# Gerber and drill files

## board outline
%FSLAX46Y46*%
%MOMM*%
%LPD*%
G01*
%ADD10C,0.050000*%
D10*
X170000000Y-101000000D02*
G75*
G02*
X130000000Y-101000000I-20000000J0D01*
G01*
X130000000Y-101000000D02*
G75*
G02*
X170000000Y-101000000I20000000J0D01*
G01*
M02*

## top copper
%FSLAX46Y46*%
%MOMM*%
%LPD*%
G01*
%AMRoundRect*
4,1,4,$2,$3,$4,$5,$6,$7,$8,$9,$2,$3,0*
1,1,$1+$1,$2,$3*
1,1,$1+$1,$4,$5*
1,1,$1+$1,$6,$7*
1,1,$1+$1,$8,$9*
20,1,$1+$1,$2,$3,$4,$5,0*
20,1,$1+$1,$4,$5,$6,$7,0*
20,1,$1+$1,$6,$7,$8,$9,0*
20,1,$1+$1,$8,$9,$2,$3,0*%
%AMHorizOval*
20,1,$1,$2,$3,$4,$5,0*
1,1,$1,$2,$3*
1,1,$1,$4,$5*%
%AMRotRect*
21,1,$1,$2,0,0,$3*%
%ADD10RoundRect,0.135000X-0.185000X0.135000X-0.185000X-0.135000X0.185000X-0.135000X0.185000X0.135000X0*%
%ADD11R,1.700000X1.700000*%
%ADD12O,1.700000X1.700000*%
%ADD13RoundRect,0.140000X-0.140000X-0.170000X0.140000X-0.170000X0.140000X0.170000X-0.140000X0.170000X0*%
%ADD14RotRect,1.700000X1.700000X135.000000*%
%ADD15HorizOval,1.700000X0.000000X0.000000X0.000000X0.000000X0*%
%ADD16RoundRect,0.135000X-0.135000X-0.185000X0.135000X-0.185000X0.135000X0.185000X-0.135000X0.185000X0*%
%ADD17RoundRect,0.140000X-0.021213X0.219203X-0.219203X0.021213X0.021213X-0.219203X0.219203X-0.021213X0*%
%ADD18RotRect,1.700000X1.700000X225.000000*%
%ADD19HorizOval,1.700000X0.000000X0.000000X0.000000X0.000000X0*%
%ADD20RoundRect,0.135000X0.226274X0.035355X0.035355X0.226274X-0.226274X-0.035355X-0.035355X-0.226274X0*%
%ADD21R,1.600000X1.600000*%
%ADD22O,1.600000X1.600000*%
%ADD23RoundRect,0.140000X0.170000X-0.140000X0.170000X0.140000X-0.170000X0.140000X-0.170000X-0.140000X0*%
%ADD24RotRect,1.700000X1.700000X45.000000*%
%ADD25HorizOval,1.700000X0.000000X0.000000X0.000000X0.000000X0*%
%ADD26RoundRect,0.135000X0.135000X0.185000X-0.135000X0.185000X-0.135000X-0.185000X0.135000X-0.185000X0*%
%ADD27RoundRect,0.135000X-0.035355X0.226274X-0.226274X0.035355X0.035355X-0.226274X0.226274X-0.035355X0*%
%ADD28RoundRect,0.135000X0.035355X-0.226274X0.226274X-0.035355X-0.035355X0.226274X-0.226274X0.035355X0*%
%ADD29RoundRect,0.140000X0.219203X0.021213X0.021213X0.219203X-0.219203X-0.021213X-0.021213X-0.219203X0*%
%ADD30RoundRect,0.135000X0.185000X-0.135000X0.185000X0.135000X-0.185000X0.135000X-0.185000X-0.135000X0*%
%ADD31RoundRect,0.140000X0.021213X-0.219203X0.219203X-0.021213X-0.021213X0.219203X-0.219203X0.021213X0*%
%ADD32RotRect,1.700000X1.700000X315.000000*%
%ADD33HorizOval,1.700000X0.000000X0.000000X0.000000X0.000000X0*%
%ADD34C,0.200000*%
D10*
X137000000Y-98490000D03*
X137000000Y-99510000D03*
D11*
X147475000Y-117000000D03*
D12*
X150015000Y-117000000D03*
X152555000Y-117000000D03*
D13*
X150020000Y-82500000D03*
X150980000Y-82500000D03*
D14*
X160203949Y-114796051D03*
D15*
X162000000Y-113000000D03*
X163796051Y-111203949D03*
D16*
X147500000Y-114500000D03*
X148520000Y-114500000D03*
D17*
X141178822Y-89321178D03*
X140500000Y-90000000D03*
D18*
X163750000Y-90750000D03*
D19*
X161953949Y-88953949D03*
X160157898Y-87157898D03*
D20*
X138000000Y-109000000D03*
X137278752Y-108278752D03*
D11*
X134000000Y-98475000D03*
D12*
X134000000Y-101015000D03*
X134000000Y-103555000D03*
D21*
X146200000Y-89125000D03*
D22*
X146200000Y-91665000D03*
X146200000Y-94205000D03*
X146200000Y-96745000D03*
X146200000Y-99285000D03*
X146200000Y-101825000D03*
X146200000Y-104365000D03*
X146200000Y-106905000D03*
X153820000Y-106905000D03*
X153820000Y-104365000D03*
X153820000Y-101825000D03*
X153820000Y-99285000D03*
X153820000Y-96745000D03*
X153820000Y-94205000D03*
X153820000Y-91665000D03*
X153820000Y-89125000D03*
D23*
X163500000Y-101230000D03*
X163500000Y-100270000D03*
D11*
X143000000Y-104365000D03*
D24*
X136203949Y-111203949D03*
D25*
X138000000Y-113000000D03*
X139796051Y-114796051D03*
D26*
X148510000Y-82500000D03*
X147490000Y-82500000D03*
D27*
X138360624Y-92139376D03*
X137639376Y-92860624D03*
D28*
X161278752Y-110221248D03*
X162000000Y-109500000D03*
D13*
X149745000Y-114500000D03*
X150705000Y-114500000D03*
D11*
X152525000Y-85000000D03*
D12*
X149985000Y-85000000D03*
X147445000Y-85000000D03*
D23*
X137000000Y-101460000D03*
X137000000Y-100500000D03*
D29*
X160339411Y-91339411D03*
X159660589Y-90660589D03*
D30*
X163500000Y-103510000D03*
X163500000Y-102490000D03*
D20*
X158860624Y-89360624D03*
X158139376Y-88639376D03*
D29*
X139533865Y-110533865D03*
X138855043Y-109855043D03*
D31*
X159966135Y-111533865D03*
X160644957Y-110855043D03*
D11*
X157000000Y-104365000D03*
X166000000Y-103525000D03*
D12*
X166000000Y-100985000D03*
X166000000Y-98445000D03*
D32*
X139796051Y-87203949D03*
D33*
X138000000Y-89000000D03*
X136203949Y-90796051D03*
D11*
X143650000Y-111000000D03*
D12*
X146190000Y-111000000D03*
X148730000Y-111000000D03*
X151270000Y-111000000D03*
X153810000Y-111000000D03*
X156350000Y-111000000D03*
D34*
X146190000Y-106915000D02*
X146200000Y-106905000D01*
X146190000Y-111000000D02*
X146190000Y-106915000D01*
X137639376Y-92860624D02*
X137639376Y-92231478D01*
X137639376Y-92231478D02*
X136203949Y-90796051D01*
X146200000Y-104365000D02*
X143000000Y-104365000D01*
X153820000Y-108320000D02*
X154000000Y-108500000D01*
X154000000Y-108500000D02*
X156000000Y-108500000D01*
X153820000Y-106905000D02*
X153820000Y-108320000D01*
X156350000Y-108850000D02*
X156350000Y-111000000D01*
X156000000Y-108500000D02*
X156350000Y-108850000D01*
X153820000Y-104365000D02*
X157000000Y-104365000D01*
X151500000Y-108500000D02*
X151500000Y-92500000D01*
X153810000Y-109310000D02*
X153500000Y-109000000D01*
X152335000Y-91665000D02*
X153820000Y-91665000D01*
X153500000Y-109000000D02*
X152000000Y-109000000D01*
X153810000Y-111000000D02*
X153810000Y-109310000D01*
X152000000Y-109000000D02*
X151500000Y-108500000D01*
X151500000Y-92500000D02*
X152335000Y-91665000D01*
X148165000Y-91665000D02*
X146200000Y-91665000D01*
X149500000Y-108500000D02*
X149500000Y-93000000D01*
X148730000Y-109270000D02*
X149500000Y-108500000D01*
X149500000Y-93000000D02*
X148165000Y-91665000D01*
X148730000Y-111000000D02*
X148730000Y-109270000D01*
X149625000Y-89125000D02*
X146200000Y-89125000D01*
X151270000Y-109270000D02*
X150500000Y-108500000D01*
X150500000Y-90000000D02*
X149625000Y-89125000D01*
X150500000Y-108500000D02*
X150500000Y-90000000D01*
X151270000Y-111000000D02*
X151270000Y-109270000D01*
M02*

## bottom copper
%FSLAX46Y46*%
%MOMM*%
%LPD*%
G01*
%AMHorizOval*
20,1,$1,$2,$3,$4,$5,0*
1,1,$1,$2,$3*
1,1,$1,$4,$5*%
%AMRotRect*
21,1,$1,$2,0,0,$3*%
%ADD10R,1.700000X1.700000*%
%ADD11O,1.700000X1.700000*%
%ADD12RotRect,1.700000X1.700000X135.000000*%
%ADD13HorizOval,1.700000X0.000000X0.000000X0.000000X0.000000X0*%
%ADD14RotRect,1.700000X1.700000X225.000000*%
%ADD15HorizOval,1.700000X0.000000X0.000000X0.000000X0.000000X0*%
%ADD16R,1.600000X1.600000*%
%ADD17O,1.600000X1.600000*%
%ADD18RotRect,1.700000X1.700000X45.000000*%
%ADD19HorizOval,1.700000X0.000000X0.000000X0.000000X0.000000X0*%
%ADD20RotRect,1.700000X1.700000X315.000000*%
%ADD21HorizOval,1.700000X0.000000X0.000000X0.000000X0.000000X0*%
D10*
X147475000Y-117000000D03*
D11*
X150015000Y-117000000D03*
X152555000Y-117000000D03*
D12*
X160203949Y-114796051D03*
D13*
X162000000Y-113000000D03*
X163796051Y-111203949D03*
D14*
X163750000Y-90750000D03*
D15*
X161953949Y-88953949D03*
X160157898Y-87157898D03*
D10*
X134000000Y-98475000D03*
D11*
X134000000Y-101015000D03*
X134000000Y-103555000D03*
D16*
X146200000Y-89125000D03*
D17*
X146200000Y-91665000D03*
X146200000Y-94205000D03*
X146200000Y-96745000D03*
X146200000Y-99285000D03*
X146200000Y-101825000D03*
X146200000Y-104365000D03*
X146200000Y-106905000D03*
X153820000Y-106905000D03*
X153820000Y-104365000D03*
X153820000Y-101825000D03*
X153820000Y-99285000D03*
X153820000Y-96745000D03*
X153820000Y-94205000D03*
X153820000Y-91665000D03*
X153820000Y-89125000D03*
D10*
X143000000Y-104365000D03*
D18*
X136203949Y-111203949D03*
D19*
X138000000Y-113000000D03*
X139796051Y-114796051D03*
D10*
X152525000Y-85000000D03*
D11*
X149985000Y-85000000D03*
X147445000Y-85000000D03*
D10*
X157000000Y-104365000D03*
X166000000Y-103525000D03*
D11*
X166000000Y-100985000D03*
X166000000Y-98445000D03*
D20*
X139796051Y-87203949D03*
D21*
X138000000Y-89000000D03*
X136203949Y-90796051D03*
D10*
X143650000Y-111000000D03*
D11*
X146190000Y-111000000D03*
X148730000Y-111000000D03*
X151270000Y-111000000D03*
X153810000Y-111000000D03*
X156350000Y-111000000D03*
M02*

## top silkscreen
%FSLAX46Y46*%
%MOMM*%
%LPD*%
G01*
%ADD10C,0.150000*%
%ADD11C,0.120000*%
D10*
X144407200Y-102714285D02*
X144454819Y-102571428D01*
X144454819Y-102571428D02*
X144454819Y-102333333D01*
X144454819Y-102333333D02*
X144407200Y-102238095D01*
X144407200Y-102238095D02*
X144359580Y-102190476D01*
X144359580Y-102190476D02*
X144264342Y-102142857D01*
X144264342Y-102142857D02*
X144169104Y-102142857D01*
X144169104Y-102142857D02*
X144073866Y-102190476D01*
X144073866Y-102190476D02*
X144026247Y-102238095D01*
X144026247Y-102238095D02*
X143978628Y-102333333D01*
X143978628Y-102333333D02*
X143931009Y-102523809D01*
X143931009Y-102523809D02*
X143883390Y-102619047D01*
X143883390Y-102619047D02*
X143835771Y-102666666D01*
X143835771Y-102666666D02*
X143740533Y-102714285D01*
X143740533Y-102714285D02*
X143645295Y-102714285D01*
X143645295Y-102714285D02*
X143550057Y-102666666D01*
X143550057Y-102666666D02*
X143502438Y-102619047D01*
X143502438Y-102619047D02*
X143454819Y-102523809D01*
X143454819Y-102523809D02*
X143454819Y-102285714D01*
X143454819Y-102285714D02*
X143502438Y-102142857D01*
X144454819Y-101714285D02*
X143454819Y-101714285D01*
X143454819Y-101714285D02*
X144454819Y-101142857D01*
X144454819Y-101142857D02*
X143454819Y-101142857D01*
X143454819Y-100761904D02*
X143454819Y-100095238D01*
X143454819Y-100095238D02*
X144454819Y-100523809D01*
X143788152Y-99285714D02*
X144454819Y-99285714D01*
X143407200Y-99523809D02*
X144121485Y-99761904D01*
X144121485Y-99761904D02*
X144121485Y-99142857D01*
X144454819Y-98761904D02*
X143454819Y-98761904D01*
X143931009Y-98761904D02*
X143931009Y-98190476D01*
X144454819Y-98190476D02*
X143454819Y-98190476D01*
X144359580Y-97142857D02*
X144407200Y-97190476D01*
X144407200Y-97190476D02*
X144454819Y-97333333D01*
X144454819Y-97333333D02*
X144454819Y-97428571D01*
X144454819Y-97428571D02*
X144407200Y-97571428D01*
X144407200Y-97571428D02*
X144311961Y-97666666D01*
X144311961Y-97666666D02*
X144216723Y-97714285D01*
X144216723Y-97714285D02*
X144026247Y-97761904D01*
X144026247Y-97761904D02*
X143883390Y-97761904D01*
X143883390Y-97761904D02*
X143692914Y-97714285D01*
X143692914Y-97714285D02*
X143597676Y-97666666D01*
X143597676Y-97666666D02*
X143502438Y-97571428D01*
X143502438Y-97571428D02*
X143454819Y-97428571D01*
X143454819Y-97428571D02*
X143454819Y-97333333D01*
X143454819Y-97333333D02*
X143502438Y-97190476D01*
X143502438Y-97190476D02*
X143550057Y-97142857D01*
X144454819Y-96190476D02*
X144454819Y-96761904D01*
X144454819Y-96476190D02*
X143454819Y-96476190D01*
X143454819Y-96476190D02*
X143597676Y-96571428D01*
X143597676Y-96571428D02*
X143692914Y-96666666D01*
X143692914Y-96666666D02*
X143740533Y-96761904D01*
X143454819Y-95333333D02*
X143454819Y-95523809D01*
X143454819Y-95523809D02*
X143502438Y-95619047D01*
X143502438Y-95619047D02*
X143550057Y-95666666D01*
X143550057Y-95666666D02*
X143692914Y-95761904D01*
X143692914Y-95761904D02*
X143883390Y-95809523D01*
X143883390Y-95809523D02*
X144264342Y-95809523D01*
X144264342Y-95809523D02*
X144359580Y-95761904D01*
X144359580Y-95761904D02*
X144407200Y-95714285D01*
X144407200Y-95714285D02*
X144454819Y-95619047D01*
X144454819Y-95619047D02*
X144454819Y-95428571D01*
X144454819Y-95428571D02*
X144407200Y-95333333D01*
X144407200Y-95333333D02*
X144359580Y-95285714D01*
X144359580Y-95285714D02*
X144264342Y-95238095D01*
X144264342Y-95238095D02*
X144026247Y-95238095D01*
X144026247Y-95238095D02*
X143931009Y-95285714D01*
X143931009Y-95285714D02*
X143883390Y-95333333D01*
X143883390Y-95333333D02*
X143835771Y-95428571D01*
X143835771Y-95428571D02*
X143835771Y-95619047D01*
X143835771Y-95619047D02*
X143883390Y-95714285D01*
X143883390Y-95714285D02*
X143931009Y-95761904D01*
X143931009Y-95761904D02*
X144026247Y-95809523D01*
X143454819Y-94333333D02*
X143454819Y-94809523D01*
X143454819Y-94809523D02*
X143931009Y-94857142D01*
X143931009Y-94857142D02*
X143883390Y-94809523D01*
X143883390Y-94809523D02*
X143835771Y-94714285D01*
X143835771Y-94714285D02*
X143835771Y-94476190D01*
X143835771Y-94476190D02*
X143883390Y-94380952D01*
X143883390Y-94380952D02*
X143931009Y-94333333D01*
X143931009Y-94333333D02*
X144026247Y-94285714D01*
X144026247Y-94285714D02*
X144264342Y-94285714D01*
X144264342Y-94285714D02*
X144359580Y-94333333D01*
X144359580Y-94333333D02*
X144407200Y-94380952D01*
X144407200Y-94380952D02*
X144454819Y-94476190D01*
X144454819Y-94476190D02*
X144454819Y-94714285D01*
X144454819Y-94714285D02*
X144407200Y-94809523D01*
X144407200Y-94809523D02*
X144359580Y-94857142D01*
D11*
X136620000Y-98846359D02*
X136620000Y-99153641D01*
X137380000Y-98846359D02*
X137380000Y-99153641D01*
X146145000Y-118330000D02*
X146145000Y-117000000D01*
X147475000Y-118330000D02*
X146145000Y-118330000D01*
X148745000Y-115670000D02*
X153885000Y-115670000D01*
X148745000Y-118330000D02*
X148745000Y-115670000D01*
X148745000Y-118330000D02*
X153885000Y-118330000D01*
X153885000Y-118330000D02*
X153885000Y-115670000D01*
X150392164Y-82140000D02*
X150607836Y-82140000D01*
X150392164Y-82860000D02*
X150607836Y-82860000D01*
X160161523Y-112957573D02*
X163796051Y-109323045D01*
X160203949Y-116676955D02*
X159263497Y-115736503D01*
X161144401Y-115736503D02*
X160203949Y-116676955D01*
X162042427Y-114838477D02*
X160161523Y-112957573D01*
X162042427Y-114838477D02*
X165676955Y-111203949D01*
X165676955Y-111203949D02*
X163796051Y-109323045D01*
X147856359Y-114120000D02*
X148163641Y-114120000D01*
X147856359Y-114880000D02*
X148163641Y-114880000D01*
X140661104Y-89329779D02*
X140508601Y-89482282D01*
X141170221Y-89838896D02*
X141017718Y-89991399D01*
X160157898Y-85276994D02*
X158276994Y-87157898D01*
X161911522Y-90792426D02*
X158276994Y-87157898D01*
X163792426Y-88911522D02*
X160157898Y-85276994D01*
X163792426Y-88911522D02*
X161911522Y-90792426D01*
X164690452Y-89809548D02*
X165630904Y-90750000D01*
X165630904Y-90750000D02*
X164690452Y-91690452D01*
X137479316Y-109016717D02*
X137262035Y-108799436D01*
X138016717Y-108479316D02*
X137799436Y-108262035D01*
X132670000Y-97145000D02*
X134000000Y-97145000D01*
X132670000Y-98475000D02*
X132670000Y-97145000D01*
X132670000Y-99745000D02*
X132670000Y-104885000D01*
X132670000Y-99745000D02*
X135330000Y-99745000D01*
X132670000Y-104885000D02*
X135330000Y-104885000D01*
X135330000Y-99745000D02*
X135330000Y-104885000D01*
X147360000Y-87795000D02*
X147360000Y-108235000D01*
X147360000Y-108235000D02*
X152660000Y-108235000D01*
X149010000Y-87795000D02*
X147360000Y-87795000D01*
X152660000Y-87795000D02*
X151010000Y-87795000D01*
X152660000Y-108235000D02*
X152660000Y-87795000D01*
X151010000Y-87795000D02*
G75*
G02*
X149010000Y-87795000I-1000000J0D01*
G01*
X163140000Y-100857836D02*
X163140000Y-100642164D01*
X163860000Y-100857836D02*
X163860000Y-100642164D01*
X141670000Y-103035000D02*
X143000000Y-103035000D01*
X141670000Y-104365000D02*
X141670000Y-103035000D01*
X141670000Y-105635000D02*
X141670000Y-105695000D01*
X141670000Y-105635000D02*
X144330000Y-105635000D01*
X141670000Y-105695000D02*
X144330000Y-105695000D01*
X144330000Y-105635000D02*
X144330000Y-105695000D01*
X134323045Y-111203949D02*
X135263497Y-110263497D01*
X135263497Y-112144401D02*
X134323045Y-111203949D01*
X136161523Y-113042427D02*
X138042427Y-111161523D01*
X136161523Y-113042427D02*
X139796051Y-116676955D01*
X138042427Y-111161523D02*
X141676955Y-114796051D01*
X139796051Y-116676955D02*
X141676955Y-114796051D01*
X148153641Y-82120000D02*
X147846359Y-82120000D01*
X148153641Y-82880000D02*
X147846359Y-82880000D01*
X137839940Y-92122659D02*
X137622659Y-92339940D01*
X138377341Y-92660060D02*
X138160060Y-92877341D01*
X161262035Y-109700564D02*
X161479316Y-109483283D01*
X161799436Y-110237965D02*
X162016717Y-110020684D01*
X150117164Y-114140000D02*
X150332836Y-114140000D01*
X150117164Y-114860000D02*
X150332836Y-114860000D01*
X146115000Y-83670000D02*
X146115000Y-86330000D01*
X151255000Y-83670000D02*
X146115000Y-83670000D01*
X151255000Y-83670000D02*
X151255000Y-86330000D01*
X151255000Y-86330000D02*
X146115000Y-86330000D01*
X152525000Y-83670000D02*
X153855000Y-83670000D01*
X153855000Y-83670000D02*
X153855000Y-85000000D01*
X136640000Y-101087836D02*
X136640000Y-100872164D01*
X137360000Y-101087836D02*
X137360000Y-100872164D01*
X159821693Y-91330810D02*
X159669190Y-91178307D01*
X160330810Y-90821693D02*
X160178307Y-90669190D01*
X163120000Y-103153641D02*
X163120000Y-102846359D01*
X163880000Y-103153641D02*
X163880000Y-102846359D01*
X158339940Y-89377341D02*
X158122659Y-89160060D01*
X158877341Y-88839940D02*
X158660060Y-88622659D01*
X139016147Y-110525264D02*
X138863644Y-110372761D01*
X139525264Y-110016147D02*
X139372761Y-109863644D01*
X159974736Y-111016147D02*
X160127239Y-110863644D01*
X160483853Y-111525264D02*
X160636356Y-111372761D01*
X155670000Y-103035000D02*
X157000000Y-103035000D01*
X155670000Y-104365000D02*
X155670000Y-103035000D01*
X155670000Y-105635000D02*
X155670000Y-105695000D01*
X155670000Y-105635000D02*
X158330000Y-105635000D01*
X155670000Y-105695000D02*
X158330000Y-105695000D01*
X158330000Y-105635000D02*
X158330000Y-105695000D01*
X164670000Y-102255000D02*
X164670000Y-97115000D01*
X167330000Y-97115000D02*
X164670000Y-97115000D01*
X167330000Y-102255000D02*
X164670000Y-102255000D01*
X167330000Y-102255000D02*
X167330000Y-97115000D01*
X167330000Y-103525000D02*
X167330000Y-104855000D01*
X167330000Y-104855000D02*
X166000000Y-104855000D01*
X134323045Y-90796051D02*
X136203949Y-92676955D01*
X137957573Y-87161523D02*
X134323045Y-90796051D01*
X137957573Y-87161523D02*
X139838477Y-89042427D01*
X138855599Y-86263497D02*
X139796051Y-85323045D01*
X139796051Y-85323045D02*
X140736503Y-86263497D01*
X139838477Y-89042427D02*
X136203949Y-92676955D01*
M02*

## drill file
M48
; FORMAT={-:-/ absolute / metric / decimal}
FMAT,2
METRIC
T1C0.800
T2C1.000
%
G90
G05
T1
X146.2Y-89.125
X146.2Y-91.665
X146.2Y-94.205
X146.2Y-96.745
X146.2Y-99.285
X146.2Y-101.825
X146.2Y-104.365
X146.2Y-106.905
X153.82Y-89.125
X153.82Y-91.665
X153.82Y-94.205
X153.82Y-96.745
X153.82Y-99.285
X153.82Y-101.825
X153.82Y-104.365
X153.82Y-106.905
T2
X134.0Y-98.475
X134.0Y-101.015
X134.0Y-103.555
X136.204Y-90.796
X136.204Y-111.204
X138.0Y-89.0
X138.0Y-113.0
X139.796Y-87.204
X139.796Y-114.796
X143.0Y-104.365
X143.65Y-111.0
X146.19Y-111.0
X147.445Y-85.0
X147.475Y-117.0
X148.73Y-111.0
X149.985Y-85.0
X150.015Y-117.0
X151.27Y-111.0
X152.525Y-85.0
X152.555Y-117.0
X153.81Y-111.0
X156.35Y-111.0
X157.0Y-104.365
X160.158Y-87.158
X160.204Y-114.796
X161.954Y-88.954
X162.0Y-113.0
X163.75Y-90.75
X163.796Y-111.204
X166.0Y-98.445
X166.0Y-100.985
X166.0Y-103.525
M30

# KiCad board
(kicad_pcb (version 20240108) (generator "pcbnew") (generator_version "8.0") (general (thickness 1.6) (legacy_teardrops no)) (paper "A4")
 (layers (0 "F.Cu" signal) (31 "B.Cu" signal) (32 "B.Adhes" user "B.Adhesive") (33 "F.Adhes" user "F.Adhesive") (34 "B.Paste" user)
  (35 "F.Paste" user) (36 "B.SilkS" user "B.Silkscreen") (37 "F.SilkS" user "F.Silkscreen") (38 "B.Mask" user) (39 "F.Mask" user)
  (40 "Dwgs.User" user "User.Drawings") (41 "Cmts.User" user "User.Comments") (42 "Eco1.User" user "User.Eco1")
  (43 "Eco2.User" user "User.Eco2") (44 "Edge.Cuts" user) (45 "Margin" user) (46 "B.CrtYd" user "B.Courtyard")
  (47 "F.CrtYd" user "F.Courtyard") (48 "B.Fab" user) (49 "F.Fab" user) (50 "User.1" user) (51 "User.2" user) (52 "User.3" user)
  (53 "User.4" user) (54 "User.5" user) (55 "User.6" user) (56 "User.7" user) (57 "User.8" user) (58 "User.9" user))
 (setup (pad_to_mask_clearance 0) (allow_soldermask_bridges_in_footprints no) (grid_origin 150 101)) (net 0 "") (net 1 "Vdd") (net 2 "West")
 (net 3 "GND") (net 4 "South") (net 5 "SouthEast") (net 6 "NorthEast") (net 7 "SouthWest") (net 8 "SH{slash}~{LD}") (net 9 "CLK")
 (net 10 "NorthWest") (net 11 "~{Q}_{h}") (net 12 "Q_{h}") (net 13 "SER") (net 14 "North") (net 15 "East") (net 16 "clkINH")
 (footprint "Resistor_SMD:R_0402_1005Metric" (layer "F.Cu") (at 137 99 -90)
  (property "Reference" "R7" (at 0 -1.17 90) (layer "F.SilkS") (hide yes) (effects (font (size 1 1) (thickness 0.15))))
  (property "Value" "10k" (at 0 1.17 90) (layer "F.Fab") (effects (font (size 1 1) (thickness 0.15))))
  (fp_line (start -0.153641 0.38) (end 0.153641 0.38) (stroke (width 0.12) (type solid)) (layer "F.SilkS"))
  (fp_line (start -0.153641 -0.38) (end 0.153641 -0.38) (stroke (width 0.12) (type solid)) (layer "F.SilkS"))
  (pad "1" smd roundrect (at -0.51 0 270) (size 0.54 0.64) (layers "F.Cu" "F.Paste" "F.Mask") (roundrect_rratio 0.25) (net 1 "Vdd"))
  (pad "2" smd roundrect (at 0.51 0 270) (size 0.54 0.64) (layers "F.Cu" "F.Paste" "F.Mask") (roundrect_rratio 0.25) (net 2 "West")))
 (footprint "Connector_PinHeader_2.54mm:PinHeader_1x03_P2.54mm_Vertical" (layer "F.Cu") (at 147.475 117 90)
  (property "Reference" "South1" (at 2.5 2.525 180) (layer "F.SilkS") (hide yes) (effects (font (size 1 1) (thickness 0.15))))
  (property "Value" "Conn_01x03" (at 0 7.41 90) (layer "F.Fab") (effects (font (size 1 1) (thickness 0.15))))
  (fp_line (start -1.33 -1.33) (end 0 -1.33) (stroke (width 0.12) (type solid)) (layer "F.SilkS"))
  (fp_line (start -1.33 0) (end -1.33 -1.33) (stroke (width 0.12) (type solid)) (layer "F.SilkS"))
  (fp_line (start 1.33 1.27) (end 1.33 6.41) (stroke (width 0.12) (type solid)) (layer "F.SilkS"))
  (fp_line (start -1.33 1.27) (end 1.33 1.27) (stroke (width 0.12) (type solid)) (layer "F.SilkS"))
  (fp_line (start -1.33 1.27) (end -1.33 6.41) (stroke (width 0.12) (type solid)) (layer "F.SilkS"))
  (fp_line (start -1.33 6.41) (end 1.33 6.41) (stroke (width 0.12) (type solid)) (layer "F.SilkS"))
  (pad "1" thru_hole rect (at 0 0 90) (size 1.7 1.7) (drill 1) (layers "*.Cu" "*.Mask") (remove_unused_layers no) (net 1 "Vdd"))
  (pad "2" thru_hole oval (at 0 2.54 90) (size 1.7 1.7) (drill 1) (layers "*.Cu" "*.Mask") (remove_unused_layers no) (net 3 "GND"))
  (pad "3" thru_hole oval (at 0 5.08 90) (size 1.7 1.7) (drill 1) (layers "*.Cu" "*.Mask") (remove_unused_layers no) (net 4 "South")))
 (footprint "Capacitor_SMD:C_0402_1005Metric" (layer "F.Cu") (at 150.5 82.5)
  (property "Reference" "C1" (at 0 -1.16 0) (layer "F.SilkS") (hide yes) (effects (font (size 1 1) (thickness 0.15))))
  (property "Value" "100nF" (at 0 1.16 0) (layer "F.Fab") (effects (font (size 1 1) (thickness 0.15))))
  (fp_line (start -0.107836 -0.36) (end 0.107836 -0.36) (stroke (width 0.12) (type solid)) (layer "F.SilkS"))
  (fp_line (start -0.107836 0.36) (end 0.107836 0.36) (stroke (width 0.12) (type solid)) (layer "F.SilkS"))
  (pad "1" smd roundrect (at -0.48 0) (size 0.56 0.62) (layers "F.Cu" "F.Paste" "F.Mask") (roundrect_rratio 0.25) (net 3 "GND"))
  (pad "2" smd roundrect (at 0.48 0) (size 0.56 0.62) (layers "F.Cu" "F.Paste" "F.Mask") (roundrect_rratio 0.25) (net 1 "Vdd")))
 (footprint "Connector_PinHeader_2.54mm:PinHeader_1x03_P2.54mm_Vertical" (layer "F.Cu") (at 160.203949 114.796051 135)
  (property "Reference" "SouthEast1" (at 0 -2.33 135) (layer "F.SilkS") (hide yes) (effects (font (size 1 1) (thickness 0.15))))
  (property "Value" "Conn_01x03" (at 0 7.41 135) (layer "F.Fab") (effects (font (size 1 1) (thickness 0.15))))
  (fp_line (start 1.33 1.270001) (end 1.33 6.409999) (stroke (width 0.12) (type solid)) (layer "F.SilkS"))
  (fp_line (start -1.33 -1.33) (end 0 -1.33) (stroke (width 0.12) (type solid)) (layer "F.SilkS"))
  (fp_line (start -1.33 0) (end -1.33 -1.33) (stroke (width 0.12) (type solid)) (layer "F.SilkS"))
  (fp_line (start -1.33 1.270001) (end 1.33 1.270001) (stroke (width 0.12) (type solid)) (layer "F.SilkS"))
  (fp_line (start -1.33 1.270001) (end -1.33 6.409999) (stroke (width 0.12) (type solid)) (layer "F.SilkS"))
  (fp_line (start -1.33 6.409999) (end 1.33 6.409999) (stroke (width 0.12) (type solid)) (layer "F.SilkS"))
  (pad "1" thru_hole rect (at 0 0 135) (size 1.7 1.7) (drill 1) (layers "*.Cu" "*.Mask") (remove_unused_layers no) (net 1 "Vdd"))
  (pad "2" thru_hole oval (at 0 2.54 135) (size 1.7 1.7) (drill 1) (layers "*.Cu" "*.Mask") (remove_unused_layers no) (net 3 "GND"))
  (pad "3" thru_hole oval (at 0 5.079999 135) (size 1.7 1.7) (drill 1) (layers "*.Cu" "*.Mask") (remove_unused_layers no)
   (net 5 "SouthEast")))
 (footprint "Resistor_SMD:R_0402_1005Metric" (layer "F.Cu") (at 148.01 114.5)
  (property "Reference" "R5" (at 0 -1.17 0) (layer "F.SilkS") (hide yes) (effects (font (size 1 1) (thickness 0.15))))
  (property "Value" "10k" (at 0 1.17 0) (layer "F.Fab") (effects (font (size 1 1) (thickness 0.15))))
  (fp_line (start -0.153641 -0.38) (end 0.153641 -0.38) (stroke (width 0.12) (type solid)) (layer "F.SilkS"))
  (fp_line (start -0.153641 0.38) (end 0.153641 0.38) (stroke (width 0.12) (type solid)) (layer "F.SilkS"))
  (pad "1" smd roundrect (at -0.51 0) (size 0.54 0.64) (layers "F.Cu" "F.Paste" "F.Mask") (roundrect_rratio 0.25) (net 1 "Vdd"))
  (pad "2" smd roundrect (at 0.51 0) (size 0.54 0.64) (layers "F.Cu" "F.Paste" "F.Mask") (roundrect_rratio 0.25) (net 4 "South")))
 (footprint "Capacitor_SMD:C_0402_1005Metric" (layer "F.Cu") (at 140.839411 89.660589 -135)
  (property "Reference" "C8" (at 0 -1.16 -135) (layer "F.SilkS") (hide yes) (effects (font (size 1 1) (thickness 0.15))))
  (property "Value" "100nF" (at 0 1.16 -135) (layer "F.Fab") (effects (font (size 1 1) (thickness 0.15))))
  (fp_line (start -0.107836 0.36) (end 0.107836 0.36) (stroke (width 0.12) (type solid)) (layer "F.SilkS"))
  (fp_line (start -0.107836 -0.36) (end 0.107836 -0.36) (stroke (width 0.12) (type solid)) (layer "F.SilkS"))
  (pad "1" smd roundrect (at -0.48 0 225) (size 0.56 0.62) (layers "F.Cu" "F.Paste" "F.Mask") (roundrect_rratio 0.25) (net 3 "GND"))
  (pad "2" smd roundrect (at 0.48 0 225) (size 0.56 0.62) (layers "F.Cu" "F.Paste" "F.Mask") (roundrect_rratio 0.25) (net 1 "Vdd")))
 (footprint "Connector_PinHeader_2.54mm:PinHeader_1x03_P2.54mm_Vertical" (layer "F.Cu") (at 163.75 90.75 -135)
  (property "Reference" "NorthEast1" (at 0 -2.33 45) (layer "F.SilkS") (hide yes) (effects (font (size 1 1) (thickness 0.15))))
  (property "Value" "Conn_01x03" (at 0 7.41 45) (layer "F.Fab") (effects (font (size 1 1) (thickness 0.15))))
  (fp_line (start -1.33 6.409999) (end 1.33 6.409999) (stroke (width 0.12) (type solid)) (layer "F.SilkS"))
  (fp_line (start 1.33 1.270001) (end 1.33 6.409999) (stroke (width 0.12) (type solid)) (layer "F.SilkS"))
  (fp_line (start -1.33 1.270001) (end -1.33 6.409999) (stroke (width 0.12) (type solid)) (layer "F.SilkS"))
  (fp_line (start -1.33 1.270001) (end 1.33 1.270001) (stroke (width 0.12) (type solid)) (layer "F.SilkS"))
  (fp_line (start -1.33 0) (end -1.33 -1.33) (stroke (width 0.12) (type solid)) (layer "F.SilkS"))
  (fp_line (start -1.33 -1.33) (end 0 -1.33) (stroke (width 0.12) (type solid)) (layer "F.SilkS"))
  (pad "1" thru_hole rect (at 0 0 225) (size 1.7 1.7) (drill 1) (layers "*.Cu" "*.Mask") (remove_unused_layers no) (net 1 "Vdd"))
  (pad "2" thru_hole oval (at 0 2.54 225) (size 1.7 1.7) (drill 1) (layers "*.Cu" "*.Mask") (remove_unused_layers no) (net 3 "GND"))
  (pad "3" thru_hole oval (at 0 5.079999 225) (size 1.7 1.7) (drill 1) (layers "*.Cu" "*.Mask") (remove_unused_layers no)
   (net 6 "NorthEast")))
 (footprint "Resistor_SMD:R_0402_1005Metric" (layer "F.Cu") (at 137.639376 108.639376 135)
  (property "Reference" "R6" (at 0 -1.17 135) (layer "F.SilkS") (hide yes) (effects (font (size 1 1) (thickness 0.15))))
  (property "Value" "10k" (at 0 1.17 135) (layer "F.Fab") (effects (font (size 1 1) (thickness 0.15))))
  (fp_line (start -0.153641 -0.38) (end 0.153641 -0.38) (stroke (width 0.12) (type solid)) (layer "F.SilkS"))
  (fp_line (start -0.153641 0.38) (end 0.153641 0.38) (stroke (width 0.12) (type solid)) (layer "F.SilkS"))
  (pad "1" smd roundrect (at -0.509999 0 135) (size 0.54 0.64) (layers "F.Cu" "F.Paste" "F.Mask") (roundrect_rratio 0.25) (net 1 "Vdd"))
  (pad "2" smd roundrect (at 0.509999 0 135) (size 0.54 0.64) (layers "F.Cu" "F.Paste" "F.Mask") (roundrect_rratio 0.25) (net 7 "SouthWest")))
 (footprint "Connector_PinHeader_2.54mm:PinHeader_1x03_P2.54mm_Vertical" (layer "F.Cu") (at 134 98.475)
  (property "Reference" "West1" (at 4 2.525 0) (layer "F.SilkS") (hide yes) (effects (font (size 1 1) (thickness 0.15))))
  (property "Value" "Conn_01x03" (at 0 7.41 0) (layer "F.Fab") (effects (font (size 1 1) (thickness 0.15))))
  (fp_line (start -1.33 -1.33) (end 0 -1.33) (stroke (width 0.12) (type solid)) (layer "F.SilkS"))
  (fp_line (start -1.33 0) (end -1.33 -1.33) (stroke (width 0.12) (type solid)) (layer "F.SilkS"))
  (fp_line (start -1.33 1.27) (end -1.33 6.41) (stroke (width 0.12) (type solid)) (layer "F.SilkS"))
  (fp_line (start -1.33 1.27) (end 1.33 1.27) (stroke (width 0.12) (type solid)) (layer "F.SilkS"))
  (fp_line (start -1.33 6.41) (end 1.33 6.41) (stroke (width 0.12) (type solid)) (layer "F.SilkS"))
  (fp_line (start 1.33 1.27) (end 1.33 6.41) (stroke (width 0.12) (type solid)) (layer "F.SilkS"))
  (pad "1" thru_hole rect (at 0 0) (size 1.7 1.7) (drill 1) (layers "*.Cu" "*.Mask") (remove_unused_layers no) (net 1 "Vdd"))
  (pad "2" thru_hole oval (at 0 2.54) (size 1.7 1.7) (drill 1) (layers "*.Cu" "*.Mask") (remove_unused_layers no) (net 3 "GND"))
  (pad "3" thru_hole oval (at 0 5.08) (size 1.7 1.7) (drill 1) (layers "*.Cu" "*.Mask") (remove_unused_layers no) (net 2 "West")))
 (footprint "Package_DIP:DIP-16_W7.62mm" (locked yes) (layer "F.Cu") (at 146.2 89.125)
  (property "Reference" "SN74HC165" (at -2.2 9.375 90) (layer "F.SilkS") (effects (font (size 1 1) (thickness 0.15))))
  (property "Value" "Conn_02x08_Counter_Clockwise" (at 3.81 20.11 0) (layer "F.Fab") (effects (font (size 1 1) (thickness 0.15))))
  (fp_line (start 1.16 -1.33) (end 1.16 19.11) (stroke (width 0.12) (type solid)) (layer "F.SilkS"))
  (fp_line (start 1.16 19.11) (end 6.46 19.11) (stroke (width 0.12) (type solid)) (layer "F.SilkS"))
  (fp_line (start 2.81 -1.33) (end 1.16 -1.33) (stroke (width 0.12) (type solid)) (layer "F.SilkS"))
  (fp_line (start 6.46 -1.33) (end 4.81 -1.33) (stroke (width 0.12) (type solid)) (layer "F.SilkS"))
  (fp_line (start 6.46 19.11) (end 6.46 -1.33) (stroke (width 0.12) (type solid)) (layer "F.SilkS"))
  (fp_arc (start 4.81 -1.33) (mid 3.81 -0.33) (end 2.81 -1.33) (stroke (width 0.12) (type solid)) (layer "F.SilkS"))
  (pad "1" thru_hole rect (at 0 0) (size 1.6 1.6) (drill 0.8) (layers "*.Cu" "*.Mask") (remove_unused_layers no) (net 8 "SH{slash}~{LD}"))
  (pad "2" thru_hole oval (at 0 2.54) (size 1.6 1.6) (drill 0.8) (layers "*.Cu" "*.Mask") (remove_unused_layers no) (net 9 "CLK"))
  (pad "3" thru_hole oval (at 0 5.08) (size 1.6 1.6) (drill 0.8) (layers "*.Cu" "*.Mask") (remove_unused_layers no) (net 6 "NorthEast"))
  (pad "4" thru_hole oval (at 0 7.62) (size 1.6 1.6) (drill 0.8) (layers "*.Cu" "*.Mask") (remove_unused_layers no) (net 5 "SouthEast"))
  (pad "5" thru_hole oval (at 0 10.16) (size 1.6 1.6) (drill 0.8) (layers "*.Cu" "*.Mask") (remove_unused_layers no) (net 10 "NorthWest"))
  (pad "6" thru_hole oval (at 0 12.7) (size 1.6 1.6) (drill 0.8) (layers "*.Cu" "*.Mask") (remove_unused_layers no) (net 7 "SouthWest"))
  (pad "7" thru_hole oval (at 0 15.24) (size 1.6 1.6) (drill 0.8) (layers "*.Cu" "*.Mask") (remove_unused_layers no) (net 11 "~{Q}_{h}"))
  (pad "8" thru_hole oval (at 0 17.78) (size 1.6 1.6) (drill 0.8) (layers "*.Cu" "*.Mask") (remove_unused_layers no) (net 3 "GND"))
  (pad "9" thru_hole oval (at 7.62 17.78) (size 1.6 1.6) (drill 0.8) (layers "*.Cu" "*.Mask") (remove_unused_layers no) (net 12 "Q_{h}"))
  (pad "10" thru_hole oval (at 7.62 15.24) (size 1.6 1.6) (drill 0.8) (layers "*.Cu" "*.Mask") (remove_unused_layers no) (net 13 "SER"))
  (pad "11" thru_hole oval (at 7.62 12.7) (size 1.6 1.6) (drill 0.8) (layers "*.Cu" "*.Mask") (remove_unused_layers no) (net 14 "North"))
  (pad "12" thru_hole oval (at 7.62 10.16) (size 1.6 1.6) (drill 0.8) (layers "*.Cu" "*.Mask") (remove_unused_layers no) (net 4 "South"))
  (pad "13" thru_hole oval (at 7.62 7.62) (size 1.6 1.6) (drill 0.8) (layers "*.Cu" "*.Mask") (remove_unused_layers no) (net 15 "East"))
  (pad "14" thru_hole oval (at 7.62 5.08) (size 1.6 1.6) (drill 0.8) (layers "*.Cu" "*.Mask") (remove_unused_layers no) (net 2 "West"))
  (pad "15" thru_hole oval (at 7.62 2.54) (size 1.6 1.6) (drill 0.8) (layers "*.Cu" "*.Mask") (remove_unused_layers no) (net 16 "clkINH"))
  (pad "16" thru_hole oval (at 7.62 0) (size 1.6 1.6) (drill 0.8) (layers "*.Cu" "*.Mask") (remove_unused_layers no) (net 1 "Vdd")))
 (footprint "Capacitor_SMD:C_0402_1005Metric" (layer "F.Cu") (at 163.5 100.75 90)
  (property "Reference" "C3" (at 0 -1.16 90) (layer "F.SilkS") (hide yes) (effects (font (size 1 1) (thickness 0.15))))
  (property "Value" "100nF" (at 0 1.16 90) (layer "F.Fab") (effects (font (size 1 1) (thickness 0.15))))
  (fp_line (start -0.107836 -0.36) (end 0.107836 -0.36) (stroke (width 0.12) (type solid)) (layer "F.SilkS"))
  (fp_line (start -0.107836 0.36) (end 0.107836 0.36) (stroke (width 0.12) (type solid)) (layer "F.SilkS"))
  (pad "1" smd roundrect (at -0.48 0 90) (size 0.56 0.62) (layers "F.Cu" "F.Paste" "F.Mask") (roundrect_rratio 0.25) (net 3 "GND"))
  (pad "2" smd roundrect (at 0.48 0 90) (size 0.56 0.62) (layers "F.Cu" "F.Paste" "F.Mask") (roundrect_rratio 0.25) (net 1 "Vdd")))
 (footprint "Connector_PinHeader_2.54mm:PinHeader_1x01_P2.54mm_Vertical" (layer "F.Cu") (at 143 104.365)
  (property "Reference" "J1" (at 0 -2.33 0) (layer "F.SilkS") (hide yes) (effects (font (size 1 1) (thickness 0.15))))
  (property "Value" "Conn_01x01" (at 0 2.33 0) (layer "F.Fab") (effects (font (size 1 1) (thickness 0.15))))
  (fp_line (start -1.33 -1.33) (end 0 -1.33) (stroke (width 0.12) (type solid)) (layer "F.SilkS"))
  (fp_line (start -1.33 0) (end -1.33 -1.33) (stroke (width 0.12) (type solid)) (layer "F.SilkS"))
  (fp_line (start -1.33 1.27) (end -1.33 1.33) (stroke (width 0.12) (type solid)) (layer "F.SilkS"))
  (fp_line (start -1.33 1.27) (end 1.33 1.27) (stroke (width 0.12) (type solid)) (layer "F.SilkS"))
  (fp_line (start -1.33 1.33) (end 1.33 1.33) (stroke (width 0.12) (type solid)) (layer "F.SilkS"))
  (fp_line (start 1.33 1.27) (end 1.33 1.33) (stroke (width 0.12) (type solid)) (layer "F.SilkS"))
  (pad "1" thru_hole rect (at 0 0) (size 1.7 1.7) (drill 1) (layers "*.Cu" "*.Mask") (remove_unused_layers no) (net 11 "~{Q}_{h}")))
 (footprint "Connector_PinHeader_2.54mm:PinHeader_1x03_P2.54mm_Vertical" (layer "F.Cu") (at 136.203949 111.203949 45)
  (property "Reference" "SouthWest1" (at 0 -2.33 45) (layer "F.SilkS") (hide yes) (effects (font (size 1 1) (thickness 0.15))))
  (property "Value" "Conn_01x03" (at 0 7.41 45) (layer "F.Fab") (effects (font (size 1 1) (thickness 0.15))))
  (fp_line (start -1.33 -1.33) (end 0 -1.33) (stroke (width 0.12) (type solid)) (layer "F.SilkS"))
  (fp_line (start -1.33 0) (end -1.33 -1.33) (stroke (width 0.12) (type solid)) (layer "F.SilkS"))
  (fp_line (start -1.33 1.270001) (end 1.33 1.270001) (stroke (width 0.12) (type solid)) (layer "F.SilkS"))
  (fp_line (start -1.33 1.270001) (end -1.33 6.409999) (stroke (width 0.12) (type solid)) (layer "F.SilkS"))
  (fp_line (start 1.33 1.270001) (end 1.33 6.409999) (stroke (width 0.12) (type solid)) (layer "F.SilkS"))
  (fp_line (start -1.33 6.409999) (end 1.33 6.409999) (stroke (width 0.12) (type solid)) (layer "F.SilkS"))
  (pad "1" thru_hole rect (at 0 0 45) (size 1.7 1.7) (drill 1) (layers "*.Cu" "*.Mask") (remove_unused_layers no) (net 1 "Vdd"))
  (pad "2" thru_hole oval (at 0 2.54 45) (size 1.7 1.7) (drill 1) (layers "*.Cu" "*.Mask") (remove_unused_layers no) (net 3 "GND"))
  (pad "3" thru_hole oval (at 0 5.079999 45) (size 1.7 1.7) (drill 1) (layers "*.Cu" "*.Mask") (remove_unused_layers no) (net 7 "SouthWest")))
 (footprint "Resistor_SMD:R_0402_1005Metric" (layer "F.Cu") (at 148 82.5 180)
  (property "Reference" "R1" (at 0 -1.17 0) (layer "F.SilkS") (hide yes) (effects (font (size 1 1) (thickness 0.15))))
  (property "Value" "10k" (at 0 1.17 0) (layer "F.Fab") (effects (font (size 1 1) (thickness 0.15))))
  (fp_line (start -0.153641 0.38) (end 0.153641 0.38) (stroke (width 0.12) (type solid)) (layer "F.SilkS"))
  (fp_line (start -0.153641 -0.38) (end 0.153641 -0.38) (stroke (width 0.12) (type solid)) (layer "F.SilkS"))
  (pad "1" smd roundrect (at -0.51 0 180) (size 0.54 0.64) (layers "F.Cu" "F.Paste" "F.Mask") (roundrect_rratio 0.25) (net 1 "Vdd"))
  (pad "2" smd roundrect (at 0.51 0 180) (size 0.54 0.64) (layers "F.Cu" "F.Paste" "F.Mask") (roundrect_rratio 0.25) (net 14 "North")))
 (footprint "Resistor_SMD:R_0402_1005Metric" (layer "F.Cu") (at 138 92.5 -135)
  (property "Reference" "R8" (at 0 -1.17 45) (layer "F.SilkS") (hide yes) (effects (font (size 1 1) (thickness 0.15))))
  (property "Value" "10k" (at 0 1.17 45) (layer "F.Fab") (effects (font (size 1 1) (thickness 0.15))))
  (fp_line (start -0.153641 0.38) (end 0.153641 0.38) (stroke (width 0.12) (type solid)) (layer "F.SilkS"))
  (fp_line (start -0.153641 -0.38) (end 0.153641 -0.38) (stroke (width 0.12) (type solid)) (layer "F.SilkS"))
  (pad "1" smd roundrect (at -0.509999 0 225) (size 0.54 0.64) (layers "F.Cu" "F.Paste" "F.Mask") (roundrect_rratio 0.25) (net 1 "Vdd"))
  (pad "2" smd roundrect (at 0.509999 0 225) (size 0.54 0.64) (layers "F.Cu" "F.Paste" "F.Mask") (roundrect_rratio 0.25)
   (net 10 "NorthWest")))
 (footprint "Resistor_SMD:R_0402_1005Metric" (layer "F.Cu") (at 161.639376 109.860624 45)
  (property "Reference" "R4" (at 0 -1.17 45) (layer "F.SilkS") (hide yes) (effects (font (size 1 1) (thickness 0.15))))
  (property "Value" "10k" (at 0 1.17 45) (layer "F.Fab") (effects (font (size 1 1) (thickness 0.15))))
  (fp_line (start -0.153641 -0.38) (end 0.153641 -0.38) (stroke (width 0.12) (type solid)) (layer "F.SilkS"))
  (fp_line (start -0.153641 0.38) (end 0.153641 0.38) (stroke (width 0.12) (type solid)) (layer "F.SilkS"))
  (pad "1" smd roundrect (at -0.509999 0 45) (size 0.54 0.64) (layers "F.Cu" "F.Paste" "F.Mask") (roundrect_rratio 0.25) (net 1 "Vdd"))
  (pad "2" smd roundrect (at 0.509999 0 45) (size 0.54 0.64) (layers "F.Cu" "F.Paste" "F.Mask") (roundrect_rratio 0.25) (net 5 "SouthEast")))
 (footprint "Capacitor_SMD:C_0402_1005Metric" (layer "F.Cu") (at 150.225 114.5)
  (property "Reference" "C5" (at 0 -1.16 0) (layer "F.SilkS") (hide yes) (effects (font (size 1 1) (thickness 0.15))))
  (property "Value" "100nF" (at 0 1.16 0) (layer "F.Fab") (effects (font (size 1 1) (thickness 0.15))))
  (fp_line (start -0.107836 -0.36) (end 0.107836 -0.36) (stroke (width 0.12) (type solid)) (layer "F.SilkS"))
  (fp_line (start -0.107836 0.36) (end 0.107836 0.36) (stroke (width 0.12) (type solid)) (layer "F.SilkS"))
  (pad "1" smd roundrect (at -0.48 0) (size 0.56 0.62) (layers "F.Cu" "F.Paste" "F.Mask") (roundrect_rratio 0.25) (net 3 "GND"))
  (pad "2" smd roundrect (at 0.48 0) (size 0.56 0.62) (layers "F.Cu" "F.Paste" "F.Mask") (roundrect_rratio 0.25) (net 1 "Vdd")))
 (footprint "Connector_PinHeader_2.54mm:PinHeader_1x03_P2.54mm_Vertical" (layer "F.Cu") (at 152.525 85 -90)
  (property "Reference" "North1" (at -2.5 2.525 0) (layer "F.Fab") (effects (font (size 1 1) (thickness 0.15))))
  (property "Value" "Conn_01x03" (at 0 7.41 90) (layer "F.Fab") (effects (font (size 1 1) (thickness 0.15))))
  (fp_line (start -1.33 6.41) (end 1.33 6.41) (stroke (width 0.12) (type solid)) (layer "F.SilkS"))
  (fp_line (start -1.33 1.27) (end -1.33 6.41) (stroke (width 0.12) (type solid)) (layer "F.SilkS"))
  (fp_line (start -1.33 1.27) (end 1.33 1.27) (stroke (width 0.12) (type solid)) (layer "F.SilkS"))
  (fp_line (start 1.33 1.27) (end 1.33 6.41) (stroke (width 0.12) (type solid)) (layer "F.SilkS"))
  (fp_line (start -1.33 0) (end -1.33 -1.33) (stroke (width 0.12) (type solid)) (layer "F.SilkS"))
  (fp_line (start -1.33 -1.33) (end 0 -1.33) (stroke (width 0.12) (type solid)) (layer "F.SilkS"))
  (pad "1" thru_hole rect (at 0 0 270) (size 1.7 1.7) (drill 1) (layers "*.Cu" "*.Mask") (remove_unused_layers no) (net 1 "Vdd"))
  (pad "2" thru_hole oval (at 0 2.54 270) (size 1.7 1.7) (drill 1) (layers "*.Cu" "*.Mask") (remove_unused_layers no) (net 3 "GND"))
  (pad "3" thru_hole oval (at 0 5.08 270) (size 1.7 1.7) (drill 1) (layers "*.Cu" "*.Mask") (remove_unused_layers no) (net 14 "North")))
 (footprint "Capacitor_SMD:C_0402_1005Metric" (layer "F.Cu") (at 137 100.98 90)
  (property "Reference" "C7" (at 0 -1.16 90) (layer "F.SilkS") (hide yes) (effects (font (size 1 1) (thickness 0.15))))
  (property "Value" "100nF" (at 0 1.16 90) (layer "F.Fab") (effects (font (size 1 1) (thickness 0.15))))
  (fp_line (start -0.107836 -0.36) (end 0.107836 -0.36) (stroke (width 0.12) (type solid)) (layer "F.SilkS"))
  (fp_line (start -0.107836 0.36) (end 0.107836 0.36) (stroke (width 0.12) (type solid)) (layer "F.SilkS"))
  (pad "1" smd roundrect (at -0.48 0 90) (size 0.56 0.62) (layers "F.Cu" "F.Paste" "F.Mask") (roundrect_rratio 0.25) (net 3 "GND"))
  (pad "2" smd roundrect (at 0.48 0 90) (size 0.56 0.62) (layers "F.Cu" "F.Paste" "F.Mask") (roundrect_rratio 0.25) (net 1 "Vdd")))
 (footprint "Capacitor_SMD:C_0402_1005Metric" (layer "F.Cu") (at 160 91 135)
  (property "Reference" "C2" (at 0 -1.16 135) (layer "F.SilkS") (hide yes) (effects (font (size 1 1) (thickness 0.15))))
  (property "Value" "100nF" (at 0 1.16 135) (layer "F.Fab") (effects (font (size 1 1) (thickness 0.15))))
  (fp_line (start -0.107836 -0.36) (end 0.107836 -0.36) (stroke (width 0.12) (type solid)) (layer "F.SilkS"))
  (fp_line (start -0.107836 0.36) (end 0.107836 0.36) (stroke (width 0.12) (type solid)) (layer "F.SilkS"))
  (pad "1" smd roundrect (at -0.48 0 135) (size 0.56 0.62) (layers "F.Cu" "F.Paste" "F.Mask") (roundrect_rratio 0.25) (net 3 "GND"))
  (pad "2" smd roundrect (at 0.48 0 135) (size 0.56 0.62) (layers "F.Cu" "F.Paste" "F.Mask") (roundrect_rratio 0.25) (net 1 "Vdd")))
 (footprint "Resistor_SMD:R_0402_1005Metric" (layer "F.Cu") (at 163.5 103 90)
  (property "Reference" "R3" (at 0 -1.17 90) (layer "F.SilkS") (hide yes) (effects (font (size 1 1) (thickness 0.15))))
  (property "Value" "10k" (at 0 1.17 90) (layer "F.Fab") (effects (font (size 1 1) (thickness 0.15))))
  (fp_line (start -0.153641 -0.38) (end 0.153641 -0.38) (stroke (width 0.12) (type solid)) (layer "F.SilkS"))
  (fp_line (start -0.153641 0.38) (end 0.153641 0.38) (stroke (width 0.12) (type solid)) (layer "F.SilkS"))
  (pad "1" smd roundrect (at -0.51 0 90) (size 0.54 0.64) (layers "F.Cu" "F.Paste" "F.Mask") (roundrect_rratio 0.25) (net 1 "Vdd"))
  (pad "2" smd roundrect (at 0.51 0 90) (size 0.54 0.64) (layers "F.Cu" "F.Paste" "F.Mask") (roundrect_rratio 0.25) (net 15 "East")))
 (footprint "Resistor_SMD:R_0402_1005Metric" (layer "F.Cu") (at 158.5 89 135)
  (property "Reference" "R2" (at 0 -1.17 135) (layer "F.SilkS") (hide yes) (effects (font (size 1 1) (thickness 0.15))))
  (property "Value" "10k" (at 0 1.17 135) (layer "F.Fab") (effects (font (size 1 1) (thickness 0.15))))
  (fp_line (start -0.153641 -0.38) (end 0.153641 -0.38) (stroke (width 0.12) (type solid)) (layer "F.SilkS"))
  (fp_line (start -0.153641 0.38) (end 0.153641 0.38) (stroke (width 0.12) (type solid)) (layer "F.SilkS"))
  (pad "1" smd roundrect (at -0.509999 0 135) (size 0.54 0.64) (layers "F.Cu" "F.Paste" "F.Mask") (roundrect_rratio 0.25) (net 1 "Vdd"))
  (pad "2" smd roundrect (at 0.509999 0 135) (size 0.54 0.64) (layers "F.Cu" "F.Paste" "F.Mask") (roundrect_rratio 0.25) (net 6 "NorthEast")))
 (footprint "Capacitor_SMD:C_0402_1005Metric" (layer "F.Cu") (at 139.194454 110.194454 135)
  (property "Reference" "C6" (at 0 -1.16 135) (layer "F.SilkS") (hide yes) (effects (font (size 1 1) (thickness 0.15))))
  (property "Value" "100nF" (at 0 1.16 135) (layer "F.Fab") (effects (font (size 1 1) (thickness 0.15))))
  (fp_line (start -0.107836 -0.36) (end 0.107836 -0.36) (stroke (width 0.12) (type solid)) (layer "F.SilkS"))
  (fp_line (start -0.107836 0.36) (end 0.107836 0.36) (stroke (width 0.12) (type solid)) (layer "F.SilkS"))
  (pad "1" smd roundrect (at -0.48 0 135) (size 0.56 0.62) (layers "F.Cu" "F.Paste" "F.Mask") (roundrect_rratio 0.25) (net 3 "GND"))
  (pad "2" smd roundrect (at 0.48 0 135) (size 0.56 0.62) (layers "F.Cu" "F.Paste" "F.Mask") (roundrect_rratio 0.25) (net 1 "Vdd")))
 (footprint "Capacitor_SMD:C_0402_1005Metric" (layer "F.Cu") (at 160.305546 111.194454 45)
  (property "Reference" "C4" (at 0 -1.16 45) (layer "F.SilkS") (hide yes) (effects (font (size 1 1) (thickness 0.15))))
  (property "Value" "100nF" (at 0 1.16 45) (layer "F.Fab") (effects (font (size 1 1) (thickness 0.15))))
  (fp_line (start -0.107836 -0.36) (end 0.107836 -0.36) (stroke (width 0.12) (type solid)) (layer "F.SilkS"))
  (fp_line (start -0.107836 0.36) (end 0.107836 0.36) (stroke (width 0.12) (type solid)) (layer "F.SilkS"))
  (pad "1" smd roundrect (at -0.48 0 45) (size 0.56 0.62) (layers "F.Cu" "F.Paste" "F.Mask") (roundrect_rratio 0.25) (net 3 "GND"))
  (pad "2" smd roundrect (at 0.48 0 45) (size 0.56 0.62) (layers "F.Cu" "F.Paste" "F.Mask") (roundrect_rratio 0.25) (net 1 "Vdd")))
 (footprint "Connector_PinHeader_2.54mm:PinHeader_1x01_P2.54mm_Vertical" (layer "F.Cu") (at 157 104.365)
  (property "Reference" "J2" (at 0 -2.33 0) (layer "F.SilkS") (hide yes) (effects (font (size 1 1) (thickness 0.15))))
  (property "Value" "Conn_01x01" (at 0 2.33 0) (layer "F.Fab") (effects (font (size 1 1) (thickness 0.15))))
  (fp_line (start -1.33 -1.33) (end 0 -1.33) (stroke (width 0.12) (type solid)) (layer "F.SilkS"))
  (fp_line (start -1.33 0) (end -1.33 -1.33) (stroke (width 0.12) (type solid)) (layer "F.SilkS"))
  (fp_line (start -1.33 1.27) (end -1.33 1.33) (stroke (width 0.12) (type solid)) (layer "F.SilkS"))
  (fp_line (start -1.33 1.27) (end 1.33 1.27) (stroke (width 0.12) (type solid)) (layer "F.SilkS"))
  (fp_line (start -1.33 1.33) (end 1.33 1.33) (stroke (width 0.12) (type solid)) (layer "F.SilkS"))
  (fp_line (start 1.33 1.27) (end 1.33 1.33) (stroke (width 0.12) (type solid)) (layer "F.SilkS"))
  (pad "1" thru_hole rect (at 0 0) (size 1.7 1.7) (drill 1) (layers "*.Cu" "*.Mask") (remove_unused_layers no) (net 13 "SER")))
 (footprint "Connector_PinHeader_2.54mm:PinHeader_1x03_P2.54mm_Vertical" (layer "F.Cu") (at 166 103.525 180)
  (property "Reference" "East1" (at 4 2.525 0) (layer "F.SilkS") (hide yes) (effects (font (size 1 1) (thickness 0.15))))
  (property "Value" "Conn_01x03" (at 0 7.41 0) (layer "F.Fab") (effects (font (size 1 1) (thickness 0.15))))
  (fp_line (start 1.33 1.27) (end 1.33 6.41) (stroke (width 0.12) (type solid)) (layer "F.SilkS"))
  (fp_line (start -1.33 6.41) (end 1.33 6.41) (stroke (width 0.12) (type solid)) (layer "F.SilkS"))
  (fp_line (start -1.33 1.27) (end 1.33 1.27) (stroke (width 0.12) (type solid)) (layer "F.SilkS"))
  (fp_line (start -1.33 1.27) (end -1.33 6.41) (stroke (width 0.12) (type solid)) (layer "F.SilkS"))
  (fp_line (start -1.33 0) (end -1.33 -1.33) (stroke (width 0.12) (type solid)) (layer "F.SilkS"))
  (fp_line (start -1.33 -1.33) (end 0 -1.33) (stroke (width 0.12) (type solid)) (layer "F.SilkS"))
  (pad "1" thru_hole rect (at 0 0 180) (size 1.7 1.7) (drill 1) (layers "*.Cu" "*.Mask") (remove_unused_layers no) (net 1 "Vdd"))
  (pad "2" thru_hole oval (at 0 2.54 180) (size 1.7 1.7) (drill 1) (layers "*.Cu" "*.Mask") (remove_unused_layers no) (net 3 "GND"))
  (pad "3" thru_hole oval (at 0 5.08 180) (size 1.7 1.7) (drill 1) (layers "*.Cu" "*.Mask") (remove_unused_layers no) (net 15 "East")))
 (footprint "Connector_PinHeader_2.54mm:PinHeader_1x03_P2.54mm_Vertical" (layer "F.Cu") (at 139.796051 87.203949 -45)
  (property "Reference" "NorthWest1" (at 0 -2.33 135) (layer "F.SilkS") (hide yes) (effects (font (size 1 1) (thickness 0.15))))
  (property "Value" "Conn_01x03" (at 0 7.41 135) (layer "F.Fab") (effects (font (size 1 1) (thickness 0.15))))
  (fp_line (start -1.33 6.409999) (end 1.33 6.409999) (stroke (width 0.12) (type solid)) (layer "F.SilkS"))
  (fp_line (start -1.33 1.270001) (end -1.33 6.409999) (stroke (width 0.12) (type solid)) (layer "F.SilkS"))
  (fp_line (start -1.33 1.270001) (end 1.33 1.270001) (stroke (width 0.12) (type solid)) (layer "F.SilkS"))
  (fp_line (start -1.33 0) (end -1.33 -1.33) (stroke (width 0.12) (type solid)) (layer "F.SilkS"))
  (fp_line (start -1.33 -1.33) (end 0 -1.33) (stroke (width 0.12) (type solid)) (layer "F.SilkS"))
  (fp_line (start 1.33 1.270001) (end 1.33 6.409999) (stroke (width 0.12) (type solid)) (layer "F.SilkS"))
  (pad "1" thru_hole rect (at 0 0 315) (size 1.7 1.7) (drill 1) (layers "*.Cu" "*.Mask") (remove_unused_layers no) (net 1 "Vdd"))
  (pad "2" thru_hole oval (at 0 2.54 315) (size 1.7 1.7) (drill 1) (layers "*.Cu" "*.Mask") (remove_unused_layers no) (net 3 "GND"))
  (pad "3" thru_hole oval (at 0 5.079999 315) (size 1.7 1.7) (drill 1) (layers "*.Cu" "*.Mask") (remove_unused_layers no)
   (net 10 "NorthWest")))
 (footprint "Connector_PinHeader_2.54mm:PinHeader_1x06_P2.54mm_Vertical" (layer "B.Cu") (at 143.65 111 -90)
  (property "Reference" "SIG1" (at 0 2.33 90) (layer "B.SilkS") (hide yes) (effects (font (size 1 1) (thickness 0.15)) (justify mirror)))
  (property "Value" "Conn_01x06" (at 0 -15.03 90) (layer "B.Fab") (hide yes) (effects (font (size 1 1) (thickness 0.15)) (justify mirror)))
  (pad "1" thru_hole rect (at 0 0 270) (size 1.7 1.7) (drill 1) (layers "*.Cu" "*.Mask") (remove_unused_layers no) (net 1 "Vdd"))
  (pad "2" thru_hole oval (at 0 -2.54 270) (size 1.7 1.7) (drill 1) (layers "*.Cu" "*.Mask") (remove_unused_layers no) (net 3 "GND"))
  (pad "3" thru_hole oval (at 0 -5.08 270) (size 1.7 1.7) (drill 1) (layers "*.Cu" "*.Mask") (remove_unused_layers no) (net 9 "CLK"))
  (pad "4" thru_hole oval (at 0 -7.62 270) (size 1.7 1.7) (drill 1) (layers "*.Cu" "*.Mask") (remove_unused_layers no)
   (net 8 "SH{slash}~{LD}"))
  (pad "5" thru_hole oval (at 0 -10.16 270) (size 1.7 1.7) (drill 1) (layers "*.Cu" "*.Mask") (remove_unused_layers no) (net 16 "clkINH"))
  (pad "6" thru_hole oval (at 0 -12.7 270) (size 1.7 1.7) (drill 1) (layers "*.Cu" "*.Mask") (remove_unused_layers no) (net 12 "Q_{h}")))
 (gr_circle (center 150 101) (end 170 101) (locked yes) (stroke (width 0.05) (type default)) (fill none) (layer "Edge.Cuts"))
 (segment (start 146.19 106.915) (end 146.2 106.905) (width 0.2) (layer "F.Cu") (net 3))
 (segment (start 146.19 111) (end 146.19 106.915) (width 0.2) (layer "F.Cu") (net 3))
 (segment (start 137.639376 92.860624) (end 137.639376 92.231478) (width 0.2) (layer "F.Cu") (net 10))
 (segment (start 137.639376 92.231478) (end 136.203949 90.796051) (width 0.2) (layer "F.Cu") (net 10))
 (segment (start 146.2 104.365) (end 143 104.365) (width 0.2) (layer "F.Cu") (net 11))
 (segment (start 153.82 108.32) (end 154 108.5) (width 0.2) (layer "F.Cu") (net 12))
 (segment (start 154 108.5) (end 156 108.5) (width 0.2) (layer "F.Cu") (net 12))
 (segment (start 153.82 106.905) (end 153.82 108.32) (width 0.2) (layer "F.Cu") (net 12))
 (segment (start 156.35 108.85) (end 156.35 111) (width 0.2) (layer "F.Cu") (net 12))
 (segment (start 156 108.5) (end 156.35 108.85) (width 0.2) (layer "F.Cu") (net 12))
 (segment (start 153.82 104.365) (end 157 104.365) (width 0.2) (layer "F.Cu") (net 13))
 (segment (start 151.5 108.5) (end 151.5 92.5) (width 0.2) (layer "F.Cu") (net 16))
 (segment (start 153.81 109.31) (end 153.5 109) (width 0.2) (layer "F.Cu") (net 16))
 (segment (start 152.335 91.665) (end 153.82 91.665) (width 0.2) (layer "F.Cu") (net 16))
 (segment (start 153.5 109) (end 152 109) (width 0.2) (layer "F.Cu") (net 16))
 (segment (start 153.81 111) (end 153.81 109.31) (width 0.2) (layer "F.Cu") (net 16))
 (segment (start 152 109) (end 151.5 108.5) (width 0.2) (layer "F.Cu") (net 16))
 (segment (start 151.5 92.5) (end 152.335 91.665) (width 0.2) (layer "F.Cu") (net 16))
 (segment (start 148.165 91.665) (end 146.2 91.665) (width 0.2) (layer "F.Cu") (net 9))
 (segment (start 149.5 108.5) (end 149.5 93) (width 0.2) (layer "F.Cu") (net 9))
 (segment (start 148.73 109.27) (end 149.5 108.5) (width 0.2) (layer "F.Cu") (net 9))
 (segment (start 149.5 93) (end 148.165 91.665) (width 0.2) (layer "F.Cu") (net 9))
 (segment (start 148.73 111) (end 148.73 109.27) (width 0.2) (layer "F.Cu") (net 9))
 (segment (start 149.625 89.125) (end 146.2 89.125) (width 0.2) (layer "F.Cu") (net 8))
 (segment (start 151.27 109.27) (end 150.5 108.5) (width 0.2) (layer "F.Cu") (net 8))
 (segment (start 150.5 90) (end 149.625 89.125) (width 0.2) (layer "F.Cu") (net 8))
 (segment (start 150.5 108.5) (end 150.5 90) (width 0.2) (layer "F.Cu") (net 8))
 (segment (start 151.27 111) (end 151.27 109.27) (width 0.2) (layer "F.Cu") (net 8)))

